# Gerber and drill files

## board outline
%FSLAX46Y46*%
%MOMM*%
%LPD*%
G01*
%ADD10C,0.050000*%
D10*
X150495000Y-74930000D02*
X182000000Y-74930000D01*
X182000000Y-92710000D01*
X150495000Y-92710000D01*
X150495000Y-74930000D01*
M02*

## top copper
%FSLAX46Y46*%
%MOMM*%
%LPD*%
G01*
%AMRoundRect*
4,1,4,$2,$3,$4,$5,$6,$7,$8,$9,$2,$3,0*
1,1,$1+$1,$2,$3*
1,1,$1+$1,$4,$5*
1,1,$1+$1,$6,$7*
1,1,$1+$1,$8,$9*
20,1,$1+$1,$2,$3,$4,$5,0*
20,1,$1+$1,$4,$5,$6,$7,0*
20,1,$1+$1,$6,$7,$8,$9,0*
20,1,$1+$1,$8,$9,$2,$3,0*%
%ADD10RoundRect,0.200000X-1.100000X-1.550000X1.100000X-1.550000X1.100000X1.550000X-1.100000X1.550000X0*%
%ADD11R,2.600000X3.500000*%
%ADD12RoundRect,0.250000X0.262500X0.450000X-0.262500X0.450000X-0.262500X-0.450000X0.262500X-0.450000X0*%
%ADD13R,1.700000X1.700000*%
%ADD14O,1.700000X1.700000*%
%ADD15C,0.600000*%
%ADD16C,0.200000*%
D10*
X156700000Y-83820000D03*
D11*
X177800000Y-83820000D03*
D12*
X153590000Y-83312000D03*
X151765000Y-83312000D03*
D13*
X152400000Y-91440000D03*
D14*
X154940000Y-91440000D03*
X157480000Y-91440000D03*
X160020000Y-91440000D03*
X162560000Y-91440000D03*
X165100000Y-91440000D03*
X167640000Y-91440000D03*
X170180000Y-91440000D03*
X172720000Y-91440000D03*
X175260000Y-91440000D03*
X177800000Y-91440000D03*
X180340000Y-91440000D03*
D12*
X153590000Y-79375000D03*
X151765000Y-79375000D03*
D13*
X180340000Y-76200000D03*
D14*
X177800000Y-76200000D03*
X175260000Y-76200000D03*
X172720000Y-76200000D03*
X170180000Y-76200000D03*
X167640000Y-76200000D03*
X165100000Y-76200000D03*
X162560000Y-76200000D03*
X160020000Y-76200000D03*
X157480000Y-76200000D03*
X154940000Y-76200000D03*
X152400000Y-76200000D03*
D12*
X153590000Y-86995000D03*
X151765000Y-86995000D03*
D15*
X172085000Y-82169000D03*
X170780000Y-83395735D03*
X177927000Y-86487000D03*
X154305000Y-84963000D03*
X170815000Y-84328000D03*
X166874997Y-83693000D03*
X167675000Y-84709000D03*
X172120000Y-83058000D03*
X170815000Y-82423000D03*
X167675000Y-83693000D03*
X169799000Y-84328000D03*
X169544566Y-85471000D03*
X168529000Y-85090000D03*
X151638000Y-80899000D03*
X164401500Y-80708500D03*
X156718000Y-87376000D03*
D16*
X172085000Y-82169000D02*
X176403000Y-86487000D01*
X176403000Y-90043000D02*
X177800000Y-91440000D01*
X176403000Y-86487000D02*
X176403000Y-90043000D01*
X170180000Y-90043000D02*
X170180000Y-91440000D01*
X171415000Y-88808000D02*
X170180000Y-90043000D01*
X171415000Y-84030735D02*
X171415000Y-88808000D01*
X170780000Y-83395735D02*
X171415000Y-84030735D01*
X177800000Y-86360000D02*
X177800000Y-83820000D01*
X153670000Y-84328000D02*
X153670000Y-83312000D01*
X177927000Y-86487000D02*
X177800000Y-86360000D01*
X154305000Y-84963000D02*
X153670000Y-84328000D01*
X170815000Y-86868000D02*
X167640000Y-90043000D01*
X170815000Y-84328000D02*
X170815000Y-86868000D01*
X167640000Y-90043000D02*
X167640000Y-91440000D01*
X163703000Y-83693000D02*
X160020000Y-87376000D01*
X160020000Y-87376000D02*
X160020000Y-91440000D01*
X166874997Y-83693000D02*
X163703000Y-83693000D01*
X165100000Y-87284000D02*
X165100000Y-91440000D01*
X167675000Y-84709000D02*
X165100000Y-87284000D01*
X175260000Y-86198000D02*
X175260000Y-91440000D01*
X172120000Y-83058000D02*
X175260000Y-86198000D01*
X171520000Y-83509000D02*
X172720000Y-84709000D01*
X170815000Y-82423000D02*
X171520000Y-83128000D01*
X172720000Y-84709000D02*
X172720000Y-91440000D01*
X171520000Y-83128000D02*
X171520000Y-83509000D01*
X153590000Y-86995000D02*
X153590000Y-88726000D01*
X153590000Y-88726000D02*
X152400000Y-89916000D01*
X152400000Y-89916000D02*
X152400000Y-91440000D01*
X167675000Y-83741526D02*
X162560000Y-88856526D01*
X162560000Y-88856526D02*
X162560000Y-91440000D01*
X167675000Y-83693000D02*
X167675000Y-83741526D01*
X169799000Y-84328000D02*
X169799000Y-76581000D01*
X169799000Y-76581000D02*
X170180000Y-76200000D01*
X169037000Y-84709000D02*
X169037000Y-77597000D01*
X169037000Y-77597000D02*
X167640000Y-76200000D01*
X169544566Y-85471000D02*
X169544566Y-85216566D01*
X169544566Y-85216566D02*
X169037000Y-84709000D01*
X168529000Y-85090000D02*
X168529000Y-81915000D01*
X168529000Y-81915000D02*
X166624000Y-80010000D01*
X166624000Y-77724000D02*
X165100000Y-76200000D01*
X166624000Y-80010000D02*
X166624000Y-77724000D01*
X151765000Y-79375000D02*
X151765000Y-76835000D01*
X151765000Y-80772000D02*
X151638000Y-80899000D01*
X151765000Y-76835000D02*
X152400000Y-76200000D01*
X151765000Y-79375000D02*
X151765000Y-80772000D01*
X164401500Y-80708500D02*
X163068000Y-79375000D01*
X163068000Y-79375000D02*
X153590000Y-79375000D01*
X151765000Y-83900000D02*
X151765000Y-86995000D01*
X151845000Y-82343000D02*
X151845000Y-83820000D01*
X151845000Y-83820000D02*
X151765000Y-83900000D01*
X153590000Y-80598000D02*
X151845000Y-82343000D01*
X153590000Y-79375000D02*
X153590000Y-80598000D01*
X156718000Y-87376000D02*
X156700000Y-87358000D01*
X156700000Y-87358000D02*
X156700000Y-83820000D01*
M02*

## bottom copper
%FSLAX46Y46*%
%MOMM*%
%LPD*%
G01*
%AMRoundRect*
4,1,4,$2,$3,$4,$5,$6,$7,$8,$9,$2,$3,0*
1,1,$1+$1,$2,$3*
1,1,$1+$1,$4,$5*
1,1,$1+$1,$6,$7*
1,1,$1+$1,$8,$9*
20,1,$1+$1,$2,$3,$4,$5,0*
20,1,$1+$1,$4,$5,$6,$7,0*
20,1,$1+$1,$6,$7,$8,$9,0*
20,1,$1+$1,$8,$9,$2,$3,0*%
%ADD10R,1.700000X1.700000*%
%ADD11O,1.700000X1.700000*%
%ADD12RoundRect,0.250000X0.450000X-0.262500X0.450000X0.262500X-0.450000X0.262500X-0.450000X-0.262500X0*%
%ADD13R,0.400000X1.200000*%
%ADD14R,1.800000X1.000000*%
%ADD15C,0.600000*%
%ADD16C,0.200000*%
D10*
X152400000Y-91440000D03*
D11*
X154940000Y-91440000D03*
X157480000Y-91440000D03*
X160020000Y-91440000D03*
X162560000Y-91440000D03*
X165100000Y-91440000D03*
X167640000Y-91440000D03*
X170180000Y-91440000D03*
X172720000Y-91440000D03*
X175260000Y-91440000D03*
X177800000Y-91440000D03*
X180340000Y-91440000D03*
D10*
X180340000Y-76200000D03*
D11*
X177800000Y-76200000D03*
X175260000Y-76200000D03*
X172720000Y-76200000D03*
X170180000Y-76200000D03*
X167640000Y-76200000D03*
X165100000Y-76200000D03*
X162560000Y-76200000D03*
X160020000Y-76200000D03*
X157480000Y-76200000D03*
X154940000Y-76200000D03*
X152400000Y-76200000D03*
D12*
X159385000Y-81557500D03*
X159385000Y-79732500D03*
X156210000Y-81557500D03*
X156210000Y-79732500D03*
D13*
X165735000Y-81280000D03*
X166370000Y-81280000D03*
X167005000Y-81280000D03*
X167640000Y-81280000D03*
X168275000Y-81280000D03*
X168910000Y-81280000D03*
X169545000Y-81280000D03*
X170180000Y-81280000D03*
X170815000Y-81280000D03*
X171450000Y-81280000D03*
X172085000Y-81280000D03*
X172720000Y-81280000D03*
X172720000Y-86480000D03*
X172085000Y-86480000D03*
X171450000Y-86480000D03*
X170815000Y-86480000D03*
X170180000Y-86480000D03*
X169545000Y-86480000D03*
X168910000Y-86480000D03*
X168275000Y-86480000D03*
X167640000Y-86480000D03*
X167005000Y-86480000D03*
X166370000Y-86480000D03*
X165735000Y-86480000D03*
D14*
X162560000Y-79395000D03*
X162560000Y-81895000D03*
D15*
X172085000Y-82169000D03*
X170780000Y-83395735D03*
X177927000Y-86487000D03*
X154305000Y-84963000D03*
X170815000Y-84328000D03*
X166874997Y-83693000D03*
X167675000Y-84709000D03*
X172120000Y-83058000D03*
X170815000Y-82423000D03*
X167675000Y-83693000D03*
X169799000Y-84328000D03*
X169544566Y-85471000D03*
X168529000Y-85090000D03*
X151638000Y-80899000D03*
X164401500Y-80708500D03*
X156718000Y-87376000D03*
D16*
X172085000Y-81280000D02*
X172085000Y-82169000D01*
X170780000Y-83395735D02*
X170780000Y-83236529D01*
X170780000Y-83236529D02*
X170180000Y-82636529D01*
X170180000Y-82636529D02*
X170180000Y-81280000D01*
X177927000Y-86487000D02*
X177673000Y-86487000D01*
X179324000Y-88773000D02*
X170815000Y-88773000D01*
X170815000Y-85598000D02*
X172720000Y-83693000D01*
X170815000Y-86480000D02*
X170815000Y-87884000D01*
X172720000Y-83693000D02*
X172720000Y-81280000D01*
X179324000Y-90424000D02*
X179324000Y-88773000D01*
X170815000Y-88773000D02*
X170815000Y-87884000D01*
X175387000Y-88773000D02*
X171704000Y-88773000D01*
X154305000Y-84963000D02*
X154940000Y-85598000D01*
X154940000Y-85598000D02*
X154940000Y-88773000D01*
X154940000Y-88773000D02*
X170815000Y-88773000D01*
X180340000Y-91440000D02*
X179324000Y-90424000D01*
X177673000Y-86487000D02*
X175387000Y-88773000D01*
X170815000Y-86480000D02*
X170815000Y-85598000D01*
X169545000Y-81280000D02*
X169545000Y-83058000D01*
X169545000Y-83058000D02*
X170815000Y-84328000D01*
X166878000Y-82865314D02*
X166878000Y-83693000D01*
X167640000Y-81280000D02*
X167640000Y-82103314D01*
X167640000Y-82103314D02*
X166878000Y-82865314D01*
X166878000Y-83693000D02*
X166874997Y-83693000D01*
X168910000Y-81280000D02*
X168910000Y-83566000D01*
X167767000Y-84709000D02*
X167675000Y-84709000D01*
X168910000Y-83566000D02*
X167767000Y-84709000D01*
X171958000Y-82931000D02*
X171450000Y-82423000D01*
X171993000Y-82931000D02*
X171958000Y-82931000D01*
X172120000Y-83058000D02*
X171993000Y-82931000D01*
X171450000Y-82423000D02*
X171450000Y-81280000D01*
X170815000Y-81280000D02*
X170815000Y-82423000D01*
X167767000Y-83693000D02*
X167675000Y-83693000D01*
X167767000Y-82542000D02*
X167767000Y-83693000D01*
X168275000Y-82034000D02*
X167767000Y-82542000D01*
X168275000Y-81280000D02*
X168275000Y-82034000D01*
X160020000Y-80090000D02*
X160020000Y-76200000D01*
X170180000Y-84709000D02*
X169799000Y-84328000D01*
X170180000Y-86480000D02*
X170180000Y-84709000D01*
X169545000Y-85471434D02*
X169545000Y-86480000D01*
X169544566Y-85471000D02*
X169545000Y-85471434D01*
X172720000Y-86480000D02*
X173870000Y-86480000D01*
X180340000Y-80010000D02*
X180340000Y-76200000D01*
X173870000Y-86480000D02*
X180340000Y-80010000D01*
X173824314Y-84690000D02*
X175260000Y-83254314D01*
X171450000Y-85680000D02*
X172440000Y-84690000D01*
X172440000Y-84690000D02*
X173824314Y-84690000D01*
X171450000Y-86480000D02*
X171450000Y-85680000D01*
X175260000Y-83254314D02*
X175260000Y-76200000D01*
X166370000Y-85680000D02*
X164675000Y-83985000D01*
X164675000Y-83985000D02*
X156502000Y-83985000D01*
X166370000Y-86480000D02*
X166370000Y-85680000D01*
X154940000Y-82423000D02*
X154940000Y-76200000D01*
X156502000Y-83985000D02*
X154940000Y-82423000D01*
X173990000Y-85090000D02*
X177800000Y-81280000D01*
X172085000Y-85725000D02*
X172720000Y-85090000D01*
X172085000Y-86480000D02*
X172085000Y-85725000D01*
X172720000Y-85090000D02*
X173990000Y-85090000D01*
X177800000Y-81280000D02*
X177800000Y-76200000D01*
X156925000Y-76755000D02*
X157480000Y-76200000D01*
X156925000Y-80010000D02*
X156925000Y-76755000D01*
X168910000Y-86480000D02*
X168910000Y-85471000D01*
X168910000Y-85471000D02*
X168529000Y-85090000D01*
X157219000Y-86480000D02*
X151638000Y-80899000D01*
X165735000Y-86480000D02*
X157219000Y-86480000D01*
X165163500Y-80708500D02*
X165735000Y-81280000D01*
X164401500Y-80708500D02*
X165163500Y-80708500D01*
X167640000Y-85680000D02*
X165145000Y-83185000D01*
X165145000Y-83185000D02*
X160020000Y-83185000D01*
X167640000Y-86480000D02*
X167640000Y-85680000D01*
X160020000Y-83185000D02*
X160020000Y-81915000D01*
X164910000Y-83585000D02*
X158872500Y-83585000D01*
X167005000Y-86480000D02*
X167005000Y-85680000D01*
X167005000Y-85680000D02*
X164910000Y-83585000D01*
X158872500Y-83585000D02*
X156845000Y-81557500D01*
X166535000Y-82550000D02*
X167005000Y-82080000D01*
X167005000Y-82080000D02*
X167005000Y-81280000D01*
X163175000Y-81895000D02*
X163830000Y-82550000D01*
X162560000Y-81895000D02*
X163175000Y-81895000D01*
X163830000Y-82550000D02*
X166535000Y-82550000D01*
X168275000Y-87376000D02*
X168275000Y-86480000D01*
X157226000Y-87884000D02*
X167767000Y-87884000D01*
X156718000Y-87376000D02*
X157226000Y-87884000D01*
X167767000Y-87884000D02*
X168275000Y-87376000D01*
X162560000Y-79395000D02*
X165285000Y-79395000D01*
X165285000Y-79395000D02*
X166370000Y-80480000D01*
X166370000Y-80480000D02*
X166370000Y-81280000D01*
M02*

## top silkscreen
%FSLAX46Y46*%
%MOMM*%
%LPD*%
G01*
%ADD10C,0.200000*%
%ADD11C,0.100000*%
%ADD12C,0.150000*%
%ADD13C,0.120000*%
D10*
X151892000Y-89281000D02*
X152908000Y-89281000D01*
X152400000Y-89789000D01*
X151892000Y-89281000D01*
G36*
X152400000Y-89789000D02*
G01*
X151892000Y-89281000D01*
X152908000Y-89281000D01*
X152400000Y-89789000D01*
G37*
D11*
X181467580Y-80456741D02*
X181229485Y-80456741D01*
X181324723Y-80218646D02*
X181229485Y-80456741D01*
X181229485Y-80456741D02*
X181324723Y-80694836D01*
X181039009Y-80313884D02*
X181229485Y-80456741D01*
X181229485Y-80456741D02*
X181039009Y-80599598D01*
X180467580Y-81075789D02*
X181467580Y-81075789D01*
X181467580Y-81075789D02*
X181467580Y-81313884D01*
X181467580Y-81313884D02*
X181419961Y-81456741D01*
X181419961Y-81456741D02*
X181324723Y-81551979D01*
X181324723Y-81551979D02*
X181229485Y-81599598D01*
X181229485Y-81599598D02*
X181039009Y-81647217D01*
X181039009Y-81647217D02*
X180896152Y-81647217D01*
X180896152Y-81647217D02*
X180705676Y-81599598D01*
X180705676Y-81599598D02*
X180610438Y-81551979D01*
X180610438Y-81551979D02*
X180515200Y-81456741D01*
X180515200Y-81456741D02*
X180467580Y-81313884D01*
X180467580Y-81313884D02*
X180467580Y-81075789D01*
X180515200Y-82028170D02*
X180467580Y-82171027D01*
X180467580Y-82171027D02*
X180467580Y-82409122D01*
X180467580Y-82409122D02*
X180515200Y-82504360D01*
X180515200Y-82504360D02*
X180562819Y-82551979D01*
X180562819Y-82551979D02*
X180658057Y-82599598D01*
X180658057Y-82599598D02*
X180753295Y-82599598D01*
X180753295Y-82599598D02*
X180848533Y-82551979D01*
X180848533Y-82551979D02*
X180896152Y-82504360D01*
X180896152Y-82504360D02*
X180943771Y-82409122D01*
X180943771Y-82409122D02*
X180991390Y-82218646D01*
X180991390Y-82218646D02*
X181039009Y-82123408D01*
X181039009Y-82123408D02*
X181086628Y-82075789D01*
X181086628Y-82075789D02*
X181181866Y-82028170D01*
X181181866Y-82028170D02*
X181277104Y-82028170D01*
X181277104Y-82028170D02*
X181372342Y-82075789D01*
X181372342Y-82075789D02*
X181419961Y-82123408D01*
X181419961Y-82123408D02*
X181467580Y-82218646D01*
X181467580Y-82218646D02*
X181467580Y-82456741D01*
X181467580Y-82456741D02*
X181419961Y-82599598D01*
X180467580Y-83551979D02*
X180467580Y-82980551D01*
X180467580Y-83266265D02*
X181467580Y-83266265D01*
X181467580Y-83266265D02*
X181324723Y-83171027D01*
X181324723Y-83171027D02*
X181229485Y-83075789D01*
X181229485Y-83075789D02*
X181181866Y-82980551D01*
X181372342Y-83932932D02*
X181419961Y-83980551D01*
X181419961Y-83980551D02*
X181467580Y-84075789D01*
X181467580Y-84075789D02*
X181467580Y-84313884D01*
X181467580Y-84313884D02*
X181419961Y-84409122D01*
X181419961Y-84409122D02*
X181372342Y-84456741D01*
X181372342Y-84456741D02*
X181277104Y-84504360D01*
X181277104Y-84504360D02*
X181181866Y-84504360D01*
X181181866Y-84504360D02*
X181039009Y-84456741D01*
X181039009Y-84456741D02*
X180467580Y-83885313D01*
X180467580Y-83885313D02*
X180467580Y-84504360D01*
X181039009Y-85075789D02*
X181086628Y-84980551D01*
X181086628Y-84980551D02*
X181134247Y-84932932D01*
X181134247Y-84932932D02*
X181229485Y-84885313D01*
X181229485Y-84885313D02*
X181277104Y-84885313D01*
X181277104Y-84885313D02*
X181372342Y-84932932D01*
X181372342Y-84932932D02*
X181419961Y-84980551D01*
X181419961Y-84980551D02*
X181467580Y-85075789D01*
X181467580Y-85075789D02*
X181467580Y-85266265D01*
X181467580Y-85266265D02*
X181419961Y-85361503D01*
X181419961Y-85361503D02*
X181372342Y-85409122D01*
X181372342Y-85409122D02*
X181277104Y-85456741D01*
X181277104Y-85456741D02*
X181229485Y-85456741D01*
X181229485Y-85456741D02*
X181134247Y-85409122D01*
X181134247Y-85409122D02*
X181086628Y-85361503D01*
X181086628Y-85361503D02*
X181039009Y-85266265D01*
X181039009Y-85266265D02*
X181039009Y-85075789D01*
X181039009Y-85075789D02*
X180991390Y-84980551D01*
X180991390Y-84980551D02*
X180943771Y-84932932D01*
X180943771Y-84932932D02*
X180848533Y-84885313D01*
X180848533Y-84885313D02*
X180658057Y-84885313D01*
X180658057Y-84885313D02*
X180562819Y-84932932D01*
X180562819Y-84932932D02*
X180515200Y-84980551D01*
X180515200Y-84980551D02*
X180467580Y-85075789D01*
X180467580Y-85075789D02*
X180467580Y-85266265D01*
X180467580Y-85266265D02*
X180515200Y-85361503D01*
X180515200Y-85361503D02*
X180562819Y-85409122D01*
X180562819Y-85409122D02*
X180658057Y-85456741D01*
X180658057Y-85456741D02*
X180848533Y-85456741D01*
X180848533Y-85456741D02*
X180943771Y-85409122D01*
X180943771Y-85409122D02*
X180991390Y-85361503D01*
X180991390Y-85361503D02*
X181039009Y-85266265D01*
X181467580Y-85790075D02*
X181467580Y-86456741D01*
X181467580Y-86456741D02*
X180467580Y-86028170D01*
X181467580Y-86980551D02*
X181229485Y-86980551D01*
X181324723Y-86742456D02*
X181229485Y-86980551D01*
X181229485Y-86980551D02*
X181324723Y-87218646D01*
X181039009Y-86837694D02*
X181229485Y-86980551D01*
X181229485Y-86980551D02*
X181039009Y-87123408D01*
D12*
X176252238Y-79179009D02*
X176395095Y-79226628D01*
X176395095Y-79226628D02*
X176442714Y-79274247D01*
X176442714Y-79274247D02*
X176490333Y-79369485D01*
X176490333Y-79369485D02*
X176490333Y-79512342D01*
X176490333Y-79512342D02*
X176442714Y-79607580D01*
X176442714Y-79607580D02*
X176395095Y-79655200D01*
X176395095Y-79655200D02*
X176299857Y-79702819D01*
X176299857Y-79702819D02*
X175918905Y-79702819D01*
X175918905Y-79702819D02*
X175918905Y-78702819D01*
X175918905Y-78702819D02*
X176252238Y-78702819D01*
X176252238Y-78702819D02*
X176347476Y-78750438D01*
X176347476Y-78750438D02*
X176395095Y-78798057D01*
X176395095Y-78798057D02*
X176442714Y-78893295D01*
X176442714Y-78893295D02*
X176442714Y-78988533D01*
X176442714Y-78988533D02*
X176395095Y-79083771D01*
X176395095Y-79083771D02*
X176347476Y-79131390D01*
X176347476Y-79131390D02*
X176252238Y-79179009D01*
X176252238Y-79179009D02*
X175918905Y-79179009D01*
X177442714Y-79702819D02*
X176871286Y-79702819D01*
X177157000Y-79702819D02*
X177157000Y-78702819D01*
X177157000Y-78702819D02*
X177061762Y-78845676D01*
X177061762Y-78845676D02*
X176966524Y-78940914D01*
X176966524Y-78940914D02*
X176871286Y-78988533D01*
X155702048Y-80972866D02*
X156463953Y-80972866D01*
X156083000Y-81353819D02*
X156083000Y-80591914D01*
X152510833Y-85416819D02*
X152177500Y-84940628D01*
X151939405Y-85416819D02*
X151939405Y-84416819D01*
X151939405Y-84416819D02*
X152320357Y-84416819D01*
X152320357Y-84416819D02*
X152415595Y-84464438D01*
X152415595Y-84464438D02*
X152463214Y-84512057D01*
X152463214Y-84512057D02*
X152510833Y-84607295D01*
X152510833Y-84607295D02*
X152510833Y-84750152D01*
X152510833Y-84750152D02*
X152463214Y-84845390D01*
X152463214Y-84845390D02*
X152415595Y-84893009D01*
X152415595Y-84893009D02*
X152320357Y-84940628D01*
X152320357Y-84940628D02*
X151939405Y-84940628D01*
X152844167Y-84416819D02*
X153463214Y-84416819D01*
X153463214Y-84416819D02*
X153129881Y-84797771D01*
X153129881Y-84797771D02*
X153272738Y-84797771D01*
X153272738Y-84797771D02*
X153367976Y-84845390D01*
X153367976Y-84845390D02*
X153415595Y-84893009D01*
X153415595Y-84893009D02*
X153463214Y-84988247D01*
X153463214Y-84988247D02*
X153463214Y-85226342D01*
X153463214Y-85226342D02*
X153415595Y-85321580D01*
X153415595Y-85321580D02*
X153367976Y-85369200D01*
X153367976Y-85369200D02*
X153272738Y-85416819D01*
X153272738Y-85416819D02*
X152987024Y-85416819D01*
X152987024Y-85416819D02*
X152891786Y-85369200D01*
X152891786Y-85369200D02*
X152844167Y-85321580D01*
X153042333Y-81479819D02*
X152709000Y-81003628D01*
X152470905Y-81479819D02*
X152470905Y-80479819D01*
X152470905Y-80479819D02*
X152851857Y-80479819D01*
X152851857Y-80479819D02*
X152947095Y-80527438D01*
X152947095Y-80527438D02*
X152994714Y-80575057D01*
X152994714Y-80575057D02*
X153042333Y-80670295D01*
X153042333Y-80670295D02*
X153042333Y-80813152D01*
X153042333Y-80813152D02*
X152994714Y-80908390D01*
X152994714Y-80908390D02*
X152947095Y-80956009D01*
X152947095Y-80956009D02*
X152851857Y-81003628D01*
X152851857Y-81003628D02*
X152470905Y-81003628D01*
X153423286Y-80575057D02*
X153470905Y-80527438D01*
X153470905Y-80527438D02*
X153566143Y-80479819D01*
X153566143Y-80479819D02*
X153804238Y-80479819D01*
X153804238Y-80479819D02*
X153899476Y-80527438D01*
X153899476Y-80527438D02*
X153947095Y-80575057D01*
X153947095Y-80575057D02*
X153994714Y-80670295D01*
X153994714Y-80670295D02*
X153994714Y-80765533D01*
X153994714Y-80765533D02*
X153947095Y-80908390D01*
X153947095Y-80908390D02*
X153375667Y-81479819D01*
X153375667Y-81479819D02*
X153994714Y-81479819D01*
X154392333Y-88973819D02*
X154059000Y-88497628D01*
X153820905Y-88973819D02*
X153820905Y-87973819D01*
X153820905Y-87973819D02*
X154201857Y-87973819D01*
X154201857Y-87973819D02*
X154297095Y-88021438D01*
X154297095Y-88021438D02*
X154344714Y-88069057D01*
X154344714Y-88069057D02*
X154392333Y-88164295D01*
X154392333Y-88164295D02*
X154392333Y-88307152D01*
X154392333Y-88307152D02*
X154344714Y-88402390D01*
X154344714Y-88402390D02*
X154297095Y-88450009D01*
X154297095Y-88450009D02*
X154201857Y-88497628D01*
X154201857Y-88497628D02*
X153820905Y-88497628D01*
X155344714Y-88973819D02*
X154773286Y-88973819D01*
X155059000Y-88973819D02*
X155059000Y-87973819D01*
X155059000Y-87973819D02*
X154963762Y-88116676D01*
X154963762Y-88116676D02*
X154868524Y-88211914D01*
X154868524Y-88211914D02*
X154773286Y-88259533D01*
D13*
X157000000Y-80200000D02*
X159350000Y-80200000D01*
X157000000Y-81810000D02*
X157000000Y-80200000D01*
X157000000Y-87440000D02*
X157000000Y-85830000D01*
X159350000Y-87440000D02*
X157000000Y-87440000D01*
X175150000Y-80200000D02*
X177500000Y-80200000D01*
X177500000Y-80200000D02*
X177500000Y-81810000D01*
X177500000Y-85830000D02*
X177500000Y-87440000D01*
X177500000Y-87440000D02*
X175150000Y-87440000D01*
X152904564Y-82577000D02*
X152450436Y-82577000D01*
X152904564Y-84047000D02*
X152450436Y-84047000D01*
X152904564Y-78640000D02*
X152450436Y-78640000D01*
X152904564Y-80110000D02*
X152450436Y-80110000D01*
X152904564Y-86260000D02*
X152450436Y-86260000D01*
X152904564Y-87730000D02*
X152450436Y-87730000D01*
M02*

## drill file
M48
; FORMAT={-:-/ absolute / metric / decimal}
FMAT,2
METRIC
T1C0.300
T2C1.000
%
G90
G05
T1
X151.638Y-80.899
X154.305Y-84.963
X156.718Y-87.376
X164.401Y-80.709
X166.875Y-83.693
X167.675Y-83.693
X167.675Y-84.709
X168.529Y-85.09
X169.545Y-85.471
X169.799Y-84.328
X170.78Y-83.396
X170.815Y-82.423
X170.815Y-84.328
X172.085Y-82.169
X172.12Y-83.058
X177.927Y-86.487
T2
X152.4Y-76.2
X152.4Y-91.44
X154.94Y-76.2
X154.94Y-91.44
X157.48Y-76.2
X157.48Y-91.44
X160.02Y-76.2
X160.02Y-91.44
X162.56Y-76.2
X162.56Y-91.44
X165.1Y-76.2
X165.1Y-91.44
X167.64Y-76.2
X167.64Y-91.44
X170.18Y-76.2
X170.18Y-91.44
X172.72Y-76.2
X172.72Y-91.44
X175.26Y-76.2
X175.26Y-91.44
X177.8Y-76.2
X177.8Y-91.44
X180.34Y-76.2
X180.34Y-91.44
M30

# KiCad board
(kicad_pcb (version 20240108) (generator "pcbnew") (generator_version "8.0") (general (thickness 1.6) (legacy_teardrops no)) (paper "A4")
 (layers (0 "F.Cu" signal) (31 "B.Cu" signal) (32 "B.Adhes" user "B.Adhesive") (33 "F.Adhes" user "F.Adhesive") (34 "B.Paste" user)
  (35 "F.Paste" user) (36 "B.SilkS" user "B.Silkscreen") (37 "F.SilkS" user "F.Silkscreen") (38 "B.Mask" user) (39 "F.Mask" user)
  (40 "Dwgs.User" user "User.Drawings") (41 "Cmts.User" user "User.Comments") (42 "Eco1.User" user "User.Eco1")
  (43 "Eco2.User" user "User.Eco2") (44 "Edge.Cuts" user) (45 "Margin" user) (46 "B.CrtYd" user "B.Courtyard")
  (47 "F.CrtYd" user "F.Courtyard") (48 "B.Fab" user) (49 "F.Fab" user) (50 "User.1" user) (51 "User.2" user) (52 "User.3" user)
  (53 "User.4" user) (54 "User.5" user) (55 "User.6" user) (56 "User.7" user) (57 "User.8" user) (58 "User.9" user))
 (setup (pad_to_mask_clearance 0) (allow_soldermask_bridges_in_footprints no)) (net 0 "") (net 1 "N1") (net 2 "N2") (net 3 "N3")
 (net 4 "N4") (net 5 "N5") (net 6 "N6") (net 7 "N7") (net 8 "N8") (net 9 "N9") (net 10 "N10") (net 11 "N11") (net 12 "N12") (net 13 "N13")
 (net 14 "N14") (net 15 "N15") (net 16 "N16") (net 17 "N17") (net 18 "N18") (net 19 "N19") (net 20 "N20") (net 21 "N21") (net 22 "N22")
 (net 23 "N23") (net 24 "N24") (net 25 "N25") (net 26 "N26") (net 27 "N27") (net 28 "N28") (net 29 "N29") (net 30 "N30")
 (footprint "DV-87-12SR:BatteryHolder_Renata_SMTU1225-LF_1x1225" (layer "F.Cu") (at 167.25 83.82)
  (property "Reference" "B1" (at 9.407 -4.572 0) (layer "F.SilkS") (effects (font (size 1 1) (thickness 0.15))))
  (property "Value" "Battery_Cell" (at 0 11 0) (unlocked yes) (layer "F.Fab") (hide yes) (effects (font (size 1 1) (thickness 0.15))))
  (fp_line (start -10.25 -3.62) (end -7.9 -3.62) (stroke (width 0.12) (type solid)) (layer "F.SilkS"))
  (fp_line (start -10.25 -2.01) (end -10.25 -3.62) (stroke (width 0.12) (type solid)) (layer "F.SilkS"))
  (fp_line (start -10.25 3.62) (end -10.25 2.01) (stroke (width 0.12) (type solid)) (layer "F.SilkS"))
  (fp_line (start -7.9 3.62) (end -10.25 3.62) (stroke (width 0.12) (type solid)) (layer "F.SilkS"))
  (fp_line (start 7.9 -3.62) (end 10.25 -3.62) (stroke (width 0.12) (type solid)) (layer "F.SilkS"))
  (fp_line (start 10.25 -3.62) (end 10.25 -2.01) (stroke (width 0.12) (type solid)) (layer "F.SilkS"))
  (fp_line (start 10.25 2.01) (end 10.25 3.62) (stroke (width 0.12) (type solid)) (layer "F.SilkS"))
  (fp_line (start 10.25 3.62) (end 7.9 3.62) (stroke (width 0.12) (type solid)) (layer "F.SilkS"))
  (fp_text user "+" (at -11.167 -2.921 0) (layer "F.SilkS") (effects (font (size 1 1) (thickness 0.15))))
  (pad "1" smd roundrect (at -10.55 0) (size 2.6 3.5) (layers "F.Cu" "F.Paste" "F.Mask") (roundrect_rratio 0.07692307692) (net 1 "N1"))
  (pad "2" smd rect (at 10.55 0) (size 2.6 3.5) (layers "F.Cu" "F.Paste" "F.Mask") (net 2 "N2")))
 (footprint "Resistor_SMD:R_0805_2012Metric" (layer "F.Cu") (at 152.6775 83.312 180)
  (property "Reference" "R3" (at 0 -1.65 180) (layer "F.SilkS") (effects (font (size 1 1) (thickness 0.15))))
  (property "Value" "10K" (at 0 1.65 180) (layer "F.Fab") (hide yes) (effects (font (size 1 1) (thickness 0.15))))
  (fp_line (start -0.227064 0.735) (end 0.227064 0.735) (stroke (width 0.12) (type solid)) (layer "F.SilkS"))
  (fp_line (start -0.227064 -0.735) (end 0.227064 -0.735) (stroke (width 0.12) (type solid)) (layer "F.SilkS"))
  (pad "1" smd roundrect (at -0.9125 0 180) (size 1.025 1.4) (layers "F.Cu" "F.Paste" "F.Mask") (roundrect_rratio 0.243902) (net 2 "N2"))
  (pad "2" smd roundrect (at 0.9125 0 180) (size 1.025 1.4) (layers "F.Cu" "F.Paste" "F.Mask") (roundrect_rratio 0.243902) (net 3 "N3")))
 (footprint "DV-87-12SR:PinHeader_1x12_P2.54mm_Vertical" (layer "F.Cu") (at 152.4 91.44 90)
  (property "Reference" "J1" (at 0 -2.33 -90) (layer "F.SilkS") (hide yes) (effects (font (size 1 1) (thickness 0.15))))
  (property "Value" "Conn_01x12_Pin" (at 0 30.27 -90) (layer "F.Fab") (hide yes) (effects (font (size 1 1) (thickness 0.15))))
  (pad "1" thru_hole rect (at 0 0 90) (size 1.7 1.7) (drill 1) (layers "*.Cu" "*.Mask") (remove_unused_layers no) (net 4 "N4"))
  (pad "2" thru_hole oval (at 0 2.54 90) (size 1.7 1.7) (drill 1) (layers "*.Cu" "*.Mask") (remove_unused_layers no) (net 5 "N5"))
  (pad "3" thru_hole oval (at 0 5.08 90) (size 1.7 1.7) (drill 1) (layers "*.Cu" "*.Mask") (remove_unused_layers no) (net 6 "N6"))
  (pad "4" thru_hole oval (at 0 7.62 90) (size 1.7 1.7) (drill 1) (layers "*.Cu" "*.Mask") (remove_unused_layers no) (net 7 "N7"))
  (pad "5" thru_hole oval (at 0 10.16 90) (size 1.7 1.7) (drill 1) (layers "*.Cu" "*.Mask") (remove_unused_layers no) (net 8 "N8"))
  (pad "6" thru_hole oval (at 0 12.7 90) (size 1.7 1.7) (drill 1) (layers "*.Cu" "*.Mask") (remove_unused_layers no) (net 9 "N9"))
  (pad "7" thru_hole oval (at 0 15.24 90) (size 1.7 1.7) (drill 1) (layers "*.Cu" "*.Mask") (remove_unused_layers no) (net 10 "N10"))
  (pad "8" thru_hole oval (at 0 17.78 90) (size 1.7 1.7) (drill 1) (layers "*.Cu" "*.Mask") (remove_unused_layers no) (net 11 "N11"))
  (pad "9" thru_hole oval (at 0 20.32 90) (size 1.7 1.7) (drill 1) (layers "*.Cu" "*.Mask") (remove_unused_layers no) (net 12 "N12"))
  (pad "10" thru_hole oval (at 0 22.86 90) (size 1.7 1.7) (drill 1) (layers "*.Cu" "*.Mask") (remove_unused_layers no) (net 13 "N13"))
  (pad "11" thru_hole oval (at 0 25.4 90) (size 1.7 1.7) (drill 1) (layers "*.Cu" "*.Mask") (remove_unused_layers no) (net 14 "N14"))
  (pad "12" thru_hole oval (at 0 27.94 90) (size 1.7 1.7) (drill 1) (layers "*.Cu" "*.Mask") (remove_unused_layers no) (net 2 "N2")))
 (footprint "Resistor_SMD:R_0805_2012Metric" (layer "F.Cu") (at 152.6775 79.375 180)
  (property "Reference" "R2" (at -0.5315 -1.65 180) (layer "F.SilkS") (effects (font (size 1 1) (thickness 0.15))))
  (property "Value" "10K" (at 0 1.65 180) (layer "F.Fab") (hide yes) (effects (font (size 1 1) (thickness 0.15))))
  (fp_line (start -0.227064 0.735) (end 0.227064 0.735) (stroke (width 0.12) (type solid)) (layer "F.SilkS"))
  (fp_line (start -0.227064 -0.735) (end 0.227064 -0.735) (stroke (width 0.12) (type solid)) (layer "F.SilkS"))
  (pad "1" smd roundrect (at -0.9125 0 180) (size 1.025 1.4) (layers "F.Cu" "F.Paste" "F.Mask") (roundrect_rratio 0.243902) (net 3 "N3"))
  (pad "2" smd roundrect (at 0.9125 0 180) (size 1.025 1.4) (layers "F.Cu" "F.Paste" "F.Mask") (roundrect_rratio 0.243902) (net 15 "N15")))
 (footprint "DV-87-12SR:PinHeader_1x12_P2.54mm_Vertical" (layer "F.Cu") (at 180.34 76.2 -90)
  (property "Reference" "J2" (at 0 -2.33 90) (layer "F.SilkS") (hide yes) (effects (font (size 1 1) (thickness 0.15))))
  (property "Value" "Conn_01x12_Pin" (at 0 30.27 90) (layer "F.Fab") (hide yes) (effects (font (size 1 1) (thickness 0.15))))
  (pad "1" thru_hole rect (at 0 0 270) (size 1.7 1.7) (drill 1) (layers "*.Cu" "*.Mask") (remove_unused_layers no) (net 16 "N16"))
  (pad "2" thru_hole oval (at 0 2.54 270) (size 1.7 1.7) (drill 1) (layers "*.Cu" "*.Mask") (remove_unused_layers no) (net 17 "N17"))
  (pad "3" thru_hole oval (at 0 5.08 270) (size 1.7 1.7) (drill 1) (layers "*.Cu" "*.Mask") (remove_unused_layers no) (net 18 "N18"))
  (pad "4" thru_hole oval (at 0 7.62 270) (size 1.7 1.7) (drill 1) (layers "*.Cu" "*.Mask") (remove_unused_layers no) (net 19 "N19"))
  (pad "5" thru_hole oval (at 0 10.16 270) (size 1.7 1.7) (drill 1) (layers "*.Cu" "*.Mask") (remove_unused_layers no) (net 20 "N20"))
  (pad "6" thru_hole oval (at 0 12.7 270) (size 1.7 1.7) (drill 1) (layers "*.Cu" "*.Mask") (remove_unused_layers no) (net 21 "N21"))
  (pad "7" thru_hole oval (at 0 15.24 270) (size 1.7 1.7) (drill 1) (layers "*.Cu" "*.Mask") (remove_unused_layers no) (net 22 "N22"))
  (pad "8" thru_hole oval (at 0 17.78 270) (size 1.7 1.7) (drill 1) (layers "*.Cu" "*.Mask") (remove_unused_layers no) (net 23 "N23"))
  (pad "9" thru_hole oval (at 0 20.32 270) (size 1.7 1.7) (drill 1) (layers "*.Cu" "*.Mask") (remove_unused_layers no) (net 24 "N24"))
  (pad "10" thru_hole oval (at 0 22.86 270) (size 1.7 1.7) (drill 1) (layers "*.Cu" "*.Mask") (remove_unused_layers no) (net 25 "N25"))
  (pad "11" thru_hole oval (at 0 25.4 270) (size 1.7 1.7) (drill 1) (layers "*.Cu" "*.Mask") (remove_unused_layers no) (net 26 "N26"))
  (pad "12" thru_hole oval (at 0 27.94 270) (size 1.7 1.7) (drill 1) (layers "*.Cu" "*.Mask") (remove_unused_layers no) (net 15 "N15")))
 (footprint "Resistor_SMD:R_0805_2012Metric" (layer "F.Cu") (at 152.6775 86.995 180)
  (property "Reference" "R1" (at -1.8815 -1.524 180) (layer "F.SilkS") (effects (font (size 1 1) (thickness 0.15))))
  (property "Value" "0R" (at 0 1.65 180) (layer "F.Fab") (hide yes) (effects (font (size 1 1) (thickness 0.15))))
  (fp_line (start -0.227064 0.735) (end 0.227064 0.735) (stroke (width 0.12) (type solid)) (layer "F.SilkS"))
  (fp_line (start -0.227064 -0.735) (end 0.227064 -0.735) (stroke (width 0.12) (type solid)) (layer "F.SilkS"))
  (pad "1" smd roundrect (at -0.9125 0 180) (size 1.025 1.4) (layers "F.Cu" "F.Paste" "F.Mask") (roundrect_rratio 0.243902) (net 4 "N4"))
  (pad "2" smd roundrect (at 0.9125 0 180) (size 1.025 1.4) (layers "F.Cu" "F.Paste" "F.Mask") (roundrect_rratio 0.243902) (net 3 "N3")))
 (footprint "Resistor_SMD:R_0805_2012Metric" (layer "B.Cu") (at 159.385 80.645 90)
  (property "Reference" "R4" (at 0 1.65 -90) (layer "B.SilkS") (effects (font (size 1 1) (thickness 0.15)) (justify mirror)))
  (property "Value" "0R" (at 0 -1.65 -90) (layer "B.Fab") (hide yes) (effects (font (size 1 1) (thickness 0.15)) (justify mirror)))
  (pad "1" smd roundrect (at -0.9125 0 90) (size 1.025 1.4) (layers "B.Cu" "B.Paste" "B.Mask") (roundrect_rratio 0.243902) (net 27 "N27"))
  (pad "2" smd roundrect (at 0.9125 0 90) (size 1.025 1.4) (layers "B.Cu" "B.Paste" "B.Mask") (roundrect_rratio 0.243902) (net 24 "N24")))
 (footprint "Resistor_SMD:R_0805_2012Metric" (layer "B.Cu") (at 156.21 80.645 90)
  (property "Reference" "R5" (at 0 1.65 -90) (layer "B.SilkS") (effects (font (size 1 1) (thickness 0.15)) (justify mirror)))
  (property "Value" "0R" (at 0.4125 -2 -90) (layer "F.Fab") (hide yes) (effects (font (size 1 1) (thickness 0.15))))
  (pad "1" smd roundrect (at -0.9125 0 90) (size 1.025 1.4) (layers "B.Cu" "B.Paste" "B.Mask") (roundrect_rratio 0.243902) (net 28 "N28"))
  (pad "2" smd roundrect (at 0.9125 0 90) (size 1.025 1.4) (layers "B.Cu" "B.Paste" "B.Mask") (roundrect_rratio 0.243902) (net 25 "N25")))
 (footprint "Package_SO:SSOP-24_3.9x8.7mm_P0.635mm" (layer "B.Cu") (at 169.2275 83.88 -90)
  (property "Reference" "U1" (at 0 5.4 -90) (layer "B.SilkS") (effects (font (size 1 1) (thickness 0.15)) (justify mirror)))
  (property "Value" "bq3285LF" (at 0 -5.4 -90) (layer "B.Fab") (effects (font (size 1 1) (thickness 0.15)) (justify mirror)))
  (pad "1" smd rect (at -2.6 3.4925 270) (size 1.2 0.4) (layers "B.Cu" "B.Paste" "B.Mask") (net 3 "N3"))
  (pad "2" smd rect (at -2.6 2.8575 270) (size 1.2 0.4) (layers "B.Cu" "B.Paste" "B.Mask") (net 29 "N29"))
  (pad "3" smd rect (at -2.6 2.2225 270) (size 1.2 0.4) (layers "B.Cu" "B.Paste" "B.Mask") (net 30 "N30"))
  (pad "4" smd rect (at -2.6 1.5875 270) (size 1.2 0.4) (layers "B.Cu" "B.Paste" "B.Mask") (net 7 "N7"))
  (pad "5" smd rect (at -2.6 0.9525 270) (size 1.2 0.4) (layers "B.Cu" "B.Paste" "B.Mask") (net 8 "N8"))
  (pad "6" smd rect (at -2.6 0.3175 270) (size 1.2 0.4) (layers "B.Cu" "B.Paste" "B.Mask") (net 9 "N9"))
  (pad "7" smd rect (at -2.6 -0.3175 270) (size 1.2 0.4) (layers "B.Cu" "B.Paste" "B.Mask") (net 10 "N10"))
  (pad "8" smd rect (at -2.6 -0.9525 270) (size 1.2 0.4) (layers "B.Cu" "B.Paste" "B.Mask") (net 11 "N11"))
  (pad "9" smd rect (at -2.6 -1.5875 270) (size 1.2 0.4) (layers "B.Cu" "B.Paste" "B.Mask") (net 12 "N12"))
  (pad "10" smd rect (at -2.6 -2.2225 270) (size 1.2 0.4) (layers "B.Cu" "B.Paste" "B.Mask") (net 13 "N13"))
  (pad "11" smd rect (at -2.6 -2.8575 270) (size 1.2 0.4) (layers "B.Cu" "B.Paste" "B.Mask") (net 14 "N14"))
  (pad "12" smd rect (at -2.6 -3.4925 270) (size 1.2 0.4) (layers "B.Cu" "B.Paste" "B.Mask") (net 2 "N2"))
  (pad "13" smd rect (at 2.6 -3.4925 270) (size 1.2 0.4) (layers "B.Cu" "B.Paste" "B.Mask") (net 16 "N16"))
  (pad "14" smd rect (at 2.6 -2.8575 270) (size 1.2 0.4) (layers "B.Cu" "B.Paste" "B.Mask") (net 17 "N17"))
  (pad "15" smd rect (at 2.6 -2.2225 270) (size 1.2 0.4) (layers "B.Cu" "B.Paste" "B.Mask") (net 18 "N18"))
  (pad "16" smd rect (at 2.6 -1.5875 270) (size 1.2 0.4) (layers "B.Cu" "B.Paste" "B.Mask") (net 2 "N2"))
  (pad "17" smd rect (at 2.6 -0.9525 270) (size 1.2 0.4) (layers "B.Cu" "B.Paste" "B.Mask") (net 20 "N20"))
  (pad "18" smd rect (at 2.6 -0.3175 270) (size 1.2 0.4) (layers "B.Cu" "B.Paste" "B.Mask") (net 21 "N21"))
  (pad "19" smd rect (at 2.6 0.3175 270) (size 1.2 0.4) (layers "B.Cu" "B.Paste" "B.Mask") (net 22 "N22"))
  (pad "20" smd rect (at 2.6 0.9525 270) (size 1.2 0.4) (layers "B.Cu" "B.Paste" "B.Mask") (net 1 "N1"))
  (pad "21" smd rect (at 2.6 1.5875 270) (size 1.2 0.4) (layers "B.Cu" "B.Paste" "B.Mask") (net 27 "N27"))
  (pad "22" smd rect (at 2.6 2.2225 270) (size 1.2 0.4) (layers "B.Cu" "B.Paste" "B.Mask") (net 28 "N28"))
  (pad "23" smd rect (at 2.6 2.8575 270) (size 1.2 0.4) (layers "B.Cu" "B.Paste" "B.Mask") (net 26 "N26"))
  (pad "24" smd rect (at 2.6 3.4925 270) (size 1.2 0.4) (layers "B.Cu" "B.Paste" "B.Mask") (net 15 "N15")))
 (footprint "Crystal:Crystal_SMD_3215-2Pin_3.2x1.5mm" (layer "B.Cu") (at 162.56 80.645 90)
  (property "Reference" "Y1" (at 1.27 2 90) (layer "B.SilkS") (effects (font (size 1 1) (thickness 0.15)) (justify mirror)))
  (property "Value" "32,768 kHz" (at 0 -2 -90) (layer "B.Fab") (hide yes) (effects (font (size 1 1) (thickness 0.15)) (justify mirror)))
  (pad "1" smd rect (at 1.25 0 90) (size 1 1.8) (layers "B.Cu" "B.Paste" "B.Mask") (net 29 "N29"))
  (pad "2" smd rect (at -1.25 0 90) (size 1 1.8) (layers "B.Cu" "B.Paste" "B.Mask") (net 30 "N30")))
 (gr_poly (pts (xy 151.892 89.281) (xy 152.908 89.281) (xy 152.4 89.789)) (stroke (width 0.2) (type solid)) (fill solid) (layer "F.SilkS"))
 (gr_rect (start 150.495 74.93) (end 182 92.71) (stroke (width 0.05) (type default)) (fill none) (layer "Edge.Cuts"))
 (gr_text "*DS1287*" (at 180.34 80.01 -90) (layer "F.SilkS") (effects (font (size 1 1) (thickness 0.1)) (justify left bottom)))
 (segment (start 172.085 82.169) (end 176.403 86.487) (width 0.2) (layer "F.Cu") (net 14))
 (segment (start 176.403 90.043) (end 177.8 91.44) (width 0.2) (layer "F.Cu") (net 14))
 (segment (start 176.403 86.487) (end 176.403 90.043) (width 0.2) (layer "F.Cu") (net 14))
 (via (at 172.085 82.169) (size 0.6) (drill 0.3) (layers "F.Cu" "B.Cu") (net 14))
 (segment (start 172.085 81.28) (end 172.085 82.169) (width 0.2) (layer "B.Cu") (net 14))
 (segment (start 170.18 90.043) (end 170.18 91.44) (width 0.2) (layer "F.Cu") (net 11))
 (segment (start 171.415 88.808) (end 170.18 90.043) (width 0.2) (layer "F.Cu") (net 11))
 (segment (start 171.415 84.030735) (end 171.415 88.808) (width 0.2) (layer "F.Cu") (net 11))
 (segment (start 170.78 83.395735) (end 171.415 84.030735) (width 0.2) (layer "F.Cu") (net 11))
 (via (at 170.78 83.395735) (size 0.6) (drill 0.3) (layers "F.Cu" "B.Cu") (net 11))
 (segment (start 170.78 83.395735) (end 170.78 83.236529) (width 0.2) (layer "B.Cu") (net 11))
 (segment (start 170.78 83.236529) (end 170.18 82.636529) (width 0.2) (layer "B.Cu") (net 11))
 (segment (start 170.18 82.636529) (end 170.18 81.28) (width 0.2) (layer "B.Cu") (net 11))
 (segment (start 177.8 86.36) (end 177.8 83.82) (width 0.2) (layer "F.Cu") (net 2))
 (segment (start 153.67 84.328) (end 153.67 83.312) (width 0.2) (layer "F.Cu") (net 2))
 (segment (start 177.927 86.487) (end 177.8 86.36) (width 0.2) (layer "F.Cu") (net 2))
 (segment (start 154.305 84.963) (end 153.67 84.328) (width 0.2) (layer "F.Cu") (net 2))
 (via (at 177.927 86.487) (size 0.6) (drill 0.3) (layers "F.Cu" "B.Cu") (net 2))
 (via (at 154.305 84.963) (size 0.6) (drill 0.3) (layers "F.Cu" "B.Cu") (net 2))
 (segment (start 177.927 86.487) (end 177.673 86.487) (width 0.2) (layer "B.Cu") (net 2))
 (segment (start 179.324 88.773) (end 170.815 88.773) (width 0.2) (layer "B.Cu") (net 2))
 (segment (start 170.815 85.598) (end 172.72 83.693) (width 0.2) (layer "B.Cu") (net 2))
 (segment (start 170.815 86.48) (end 170.815 87.884) (width 0.2) (layer "B.Cu") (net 2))
 (segment (start 172.72 83.693) (end 172.72 81.28) (width 0.2) (layer "B.Cu") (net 2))
 (segment (start 179.324 90.424) (end 179.324 88.773) (width 0.2) (layer "B.Cu") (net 2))
 (segment (start 170.815 88.773) (end 170.815 87.884) (width 0.2) (layer "B.Cu") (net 2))
 (segment (start 175.387 88.773) (end 171.704 88.773) (width 0.2) (layer "B.Cu") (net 2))
 (segment (start 154.305 84.963) (end 154.94 85.598) (width 0.2) (layer "B.Cu") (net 2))
 (segment (start 154.94 85.598) (end 154.94 88.773) (width 0.2) (layer "B.Cu") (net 2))
 (segment (start 154.94 88.773) (end 170.815 88.773) (width 0.2) (layer "B.Cu") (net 2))
 (segment (start 180.34 91.44) (end 179.324 90.424) (width 0.2) (layer "B.Cu") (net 2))
 (segment (start 177.673 86.487) (end 175.387 88.773) (width 0.2) (layer "B.Cu") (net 2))
 (segment (start 170.815 86.48) (end 170.815 85.598) (width 0.2) (layer "B.Cu") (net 2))
 (segment (start 170.815 86.868) (end 167.64 90.043) (width 0.2) (layer "F.Cu") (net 10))
 (segment (start 170.815 84.328) (end 170.815 86.868) (width 0.2) (layer "F.Cu") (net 10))
 (segment (start 167.64 90.043) (end 167.64 91.44) (width 0.2) (layer "F.Cu") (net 10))
 (via (at 170.815 84.328) (size 0.6) (drill 0.3) (layers "F.Cu" "B.Cu") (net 10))
 (segment (start 169.545 81.28) (end 169.545 83.058) (width 0.2) (layer "B.Cu") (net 10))
 (segment (start 169.545 83.058) (end 170.815 84.328) (width 0.2) (layer "B.Cu") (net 10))
 (segment (start 163.703 83.693) (end 160.02 87.376) (width 0.2) (layer "F.Cu") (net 7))
 (segment (start 160.02 87.376) (end 160.02 91.44) (width 0.2) (layer "F.Cu") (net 7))
 (segment (start 166.874997 83.693) (end 163.703 83.693) (width 0.2) (layer "F.Cu") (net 7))
 (via (at 166.874997 83.693) (size 0.6) (drill 0.3) (layers "F.Cu" "B.Cu") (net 7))
 (segment (start 166.878 82.865314) (end 166.878 83.693) (width 0.2) (layer "B.Cu") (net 7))
 (segment (start 167.64 81.28) (end 167.64 82.103314) (width 0.2) (layer "B.Cu") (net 7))
 (segment (start 167.64 82.103314) (end 166.878 82.865314) (width 0.2) (layer "B.Cu") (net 7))
 (segment (start 166.878 83.693) (end 166.874997 83.693) (width 0.2) (layer "B.Cu") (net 7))
 (segment (start 165.1 87.284) (end 165.1 91.44) (width 0.2) (layer "F.Cu") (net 9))
 (segment (start 167.675 84.709) (end 165.1 87.284) (width 0.2) (layer "F.Cu") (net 9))
 (via (at 167.675 84.709) (size 0.6) (drill 0.3) (layers "F.Cu" "B.Cu") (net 9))
 (segment (start 168.91 81.28) (end 168.91 83.566) (width 0.2) (layer "B.Cu") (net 9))
 (segment (start 167.767 84.709) (end 167.675 84.709) (width 0.2) (layer "B.Cu") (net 9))
 (segment (start 168.91 83.566) (end 167.767 84.709) (width 0.2) (layer "B.Cu") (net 9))
 (segment (start 175.26 86.198) (end 175.26 91.44) (width 0.2) (layer "F.Cu") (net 13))
 (segment (start 172.12 83.058) (end 175.26 86.198) (width 0.2) (layer "F.Cu") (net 13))
 (via (at 172.12 83.058) (size 0.6) (drill 0.3) (layers "F.Cu" "B.Cu") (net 13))
 (segment (start 171.958 82.931) (end 171.45 82.423) (width 0.2) (layer "B.Cu") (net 13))
 (segment (start 171.993 82.931) (end 171.958 82.931) (width 0.2) (layer "B.Cu") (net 13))
 (segment (start 172.12 83.058) (end 171.993 82.931) (width 0.2) (layer "B.Cu") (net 13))
 (segment (start 171.45 82.423) (end 171.45 81.28) (width 0.2) (layer "B.Cu") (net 13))
 (segment (start 171.52 83.509) (end 172.72 84.709) (width 0.2) (layer "F.Cu") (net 12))
 (segment (start 170.815 82.423) (end 171.52 83.128) (width 0.2) (layer "F.Cu") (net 12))
 (segment (start 172.72 84.709) (end 172.72 91.44) (width 0.2) (layer "F.Cu") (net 12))
 (segment (start 171.52 83.128) (end 171.52 83.509) (width 0.2) (layer "F.Cu") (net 12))
 (via (at 170.815 82.423) (size 0.6) (drill 0.3) (layers "F.Cu" "B.Cu") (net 12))
 (segment (start 170.815 81.28) (end 170.815 82.423) (width 0.2) (layer "B.Cu") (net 12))
 (segment (start 153.59 86.995) (end 153.59 88.726) (width 0.2) (layer "F.Cu") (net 4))
 (segment (start 153.59 88.726) (end 152.4 89.916) (width 0.2) (layer "F.Cu") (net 4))
 (segment (start 152.4 89.916) (end 152.4 91.44) (width 0.2) (layer "F.Cu") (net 4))
 (segment (start 167.675 83.741526) (end 162.56 88.856526) (width 0.2) (layer "F.Cu") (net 8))
 (segment (start 162.56 88.856526) (end 162.56 91.44) (width 0.2) (layer "F.Cu") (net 8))
 (segment (start 167.675 83.693) (end 167.675 83.741526) (width 0.2) (layer "F.Cu") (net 8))
 (via (at 167.675 83.693) (size 0.6) (drill 0.3) (layers "F.Cu" "B.Cu") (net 8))
 (segment (start 167.767 83.693) (end 167.675 83.693) (width 0.2) (layer "B.Cu") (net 8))
 (segment (start 167.767 82.542) (end 167.767 83.693) (width 0.2) (layer "B.Cu") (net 8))
 (segment (start 168.275 82.034) (end 167.767 82.542) (width 0.2) (layer "B.Cu") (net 8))
 (segment (start 168.275 81.28) (end 168.275 82.034) (width 0.2) (layer "B.Cu") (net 8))
 (segment (start 160.02 80.09) (end 160.02 76.2) (width 0.2) (layer "B.Cu") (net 24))
 (segment (start 169.799 84.328) (end 169.799 76.581) (width 0.2) (layer "F.Cu") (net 20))
 (segment (start 169.799 76.581) (end 170.18 76.2) (width 0.2) (layer "F.Cu") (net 20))
 (via (at 169.799 84.328) (size 0.6) (drill 0.3) (layers "F.Cu" "B.Cu") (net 20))
 (segment (start 170.18 84.709) (end 169.799 84.328) (width 0.2) (layer "B.Cu") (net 20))
 (segment (start 170.18 86.48) (end 170.18 84.709) (width 0.2) (layer "B.Cu") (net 20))
 (segment (start 169.037 84.709) (end 169.037 77.597) (width 0.2) (layer "F.Cu") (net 21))
 (segment (start 169.037 77.597) (end 167.64 76.2) (width 0.2) (layer "F.Cu") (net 21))
 (segment (start 169.544566 85.471) (end 169.544566 85.216566) (width 0.2) (layer "F.Cu") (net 21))
 (segment (start 169.544566 85.216566) (end 169.037 84.709) (width 0.2) (layer "F.Cu") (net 21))
 (via (at 169.544566 85.471) (size 0.6) (drill 0.3) (layers "F.Cu" "B.Cu") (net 21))
 (segment (start 169.545 85.471434) (end 169.545 86.48) (width 0.2) (layer "B.Cu") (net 21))
 (segment (start 169.544566 85.471) (end 169.545 85.471434) (width 0.2) (layer "B.Cu") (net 21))
 (segment (start 172.72 86.48) (end 173.87 86.48) (width 0.2) (layer "B.Cu") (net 16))
 (segment (start 180.34 80.01) (end 180.34 76.2) (width 0.2) (layer "B.Cu") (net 16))
 (segment (start 173.87 86.48) (end 180.34 80.01) (width 0.2) (layer "B.Cu") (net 16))
 (segment (start 173.824314 84.69) (end 175.26 83.254314) (width 0.2) (layer "B.Cu") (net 18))
 (segment (start 171.45 85.68) (end 172.44 84.69) (width 0.2) (layer "B.Cu") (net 18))
 (segment (start 172.44 84.69) (end 173.824314 84.69) (width 0.2) (layer "B.Cu") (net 18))
 (segment (start 171.45 86.48) (end 171.45 85.68) (width 0.2) (layer "B.Cu") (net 18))
 (segment (start 175.26 83.254314) (end 175.26 76.2) (width 0.2) (layer "B.Cu") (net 18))
 (segment (start 166.37 85.68) (end 164.675 83.985) (width 0.2) (layer "B.Cu") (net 26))
 (segment (start 164.675 83.985) (end 156.502 83.985) (width 0.2) (layer "B.Cu") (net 26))
 (segment (start 166.37 86.48) (end 166.37 85.68) (width 0.2) (layer "B.Cu") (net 26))
 (segment (start 154.94 82.423) (end 154.94 76.2) (width 0.2) (layer "B.Cu") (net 26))
 (segment (start 156.502 83.985) (end 154.94 82.423) (width 0.2) (layer "B.Cu") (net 26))
 (segment (start 173.99 85.09) (end 177.8 81.28) (width 0.2) (layer "B.Cu") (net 17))
 (segment (start 172.085 85.725) (end 172.72 85.09) (width 0.2) (layer "B.Cu") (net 17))
 (segment (start 172.085 86.48) (end 172.085 85.725) (width 0.2) (layer "B.Cu") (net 17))
 (segment (start 172.72 85.09) (end 173.99 85.09) (width 0.2) (layer "B.Cu") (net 17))
 (segment (start 177.8 81.28) (end 177.8 76.2) (width 0.2) (layer "B.Cu") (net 17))
 (segment (start 156.925 76.755) (end 157.48 76.2) (width 0.2) (layer "B.Cu") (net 25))
 (segment (start 156.925 80.01) (end 156.925 76.755) (width 0.2) (layer "B.Cu") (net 25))
 (segment (start 168.529 85.09) (end 168.529 81.915) (width 0.2) (layer "F.Cu") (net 22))
 (segment (start 168.529 81.915) (end 166.624 80.01) (width 0.2) (layer "F.Cu") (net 22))
 (segment (start 166.624 77.724) (end 165.1 76.2) (width 0.2) (layer "F.Cu") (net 22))
 (segment (start 166.624 80.01) (end 166.624 77.724) (width 0.2) (layer "F.Cu") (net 22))
 (via (at 168.529 85.09) (size 0.6) (drill 0.3) (layers "F.Cu" "B.Cu") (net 22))
 (segment (start 168.91 86.48) (end 168.91 85.471) (width 0.2) (layer "B.Cu") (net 22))
 (segment (start 168.91 85.471) (end 168.529 85.09) (width 0.2) (layer "B.Cu") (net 22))
 (segment (start 151.765 79.375) (end 151.765 76.835) (width 0.2) (layer "F.Cu") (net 15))
 (segment (start 151.765 80.772) (end 151.638 80.899) (width 0.2) (layer "F.Cu") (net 15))
 (segment (start 151.765 76.835) (end 152.4 76.2) (width 0.2) (layer "F.Cu") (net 15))
 (segment (start 151.765 79.375) (end 151.765 80.772) (width 0.2) (layer "F.Cu") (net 15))
 (via (at 151.638 80.899) (size 0.6) (drill 0.3) (layers "F.Cu" "B.Cu") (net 15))
 (segment (start 157.219 86.48) (end 151.638 80.899) (width 0.2) (layer "B.Cu") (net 15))
 (segment (start 165.735 86.48) (end 157.219 86.48) (width 0.2) (layer "B.Cu") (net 15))
 (segment (start 164.4015 80.7085) (end 163.068 79.375) (width 0.2) (layer "F.Cu") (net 3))
 (segment (start 163.068 79.375) (end 153.59 79.375) (width 0.2) (layer "F.Cu") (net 3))
 (segment (start 151.765 83.9) (end 151.765 86.995) (width 0.2) (layer "F.Cu") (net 3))
 (segment (start 151.845 82.343) (end 151.845 83.82) (width 0.2) (layer "F.Cu") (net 3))
 (segment (start 151.845 83.82) (end 151.765 83.9) (width 0.2) (layer "F.Cu") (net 3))
 (segment (start 153.59 80.598) (end 151.845 82.343) (width 0.2) (layer "F.Cu") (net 3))
 (segment (start 153.59 79.375) (end 153.59 80.598) (width 0.2) (layer "F.Cu") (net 3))
 (via (at 164.4015 80.7085) (size 0.6) (drill 0.3) (layers "F.Cu" "B.Cu") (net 3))
 (segment (start 165.1635 80.7085) (end 165.735 81.28) (width 0.2) (layer "B.Cu") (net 3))
 (segment (start 164.4015 80.7085) (end 165.1635 80.7085) (width 0.2) (layer "B.Cu") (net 3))
 (segment (start 167.64 85.68) (end 165.145 83.185) (width 0.2) (layer "B.Cu") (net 27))
 (segment (start 165.145 83.185) (end 160.02 83.185) (width 0.2) (layer "B.Cu") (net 27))
 (segment (start 167.64 86.48) (end 167.64 85.68) (width 0.2) (layer "B.Cu") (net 27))
 (segment (start 160.02 83.185) (end 160.02 81.915) (width 0.2) (layer "B.Cu") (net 27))
 (segment (start 164.91 83.585) (end 158.8725 83.585) (width 0.2) (layer "B.Cu") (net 28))
 (segment (start 167.005 86.48) (end 167.005 85.68) (width 0.2) (layer "B.Cu") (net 28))
 (segment (start 167.005 85.68) (end 164.91 83.585) (width 0.2) (layer "B.Cu") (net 28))
 (segment (start 158.8725 83.585) (end 156.845 81.5575) (width 0.2) (layer "B.Cu") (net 28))
 (segment (start 166.535 82.55) (end 167.005 82.08) (width 0.2) (layer "B.Cu") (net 30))
 (segment (start 167.005 82.08) (end 167.005 81.28) (width 0.2) (layer "B.Cu") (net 30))
 (segment (start 163.175 81.895) (end 163.83 82.55) (width 0.2) (layer "B.Cu") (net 30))
 (segment (start 162.56 81.895) (end 163.175 81.895) (width 0.2) (layer "B.Cu") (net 30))
 (segment (start 163.83 82.55) (end 166.535 82.55) (width 0.2) (layer "B.Cu") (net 30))
 (segment (start 156.718 87.376) (end 156.7 87.358) (width 0.2) (layer "F.Cu") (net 1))
 (segment (start 156.7 87.358) (end 156.7 83.82) (width 0.2) (layer "F.Cu") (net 1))
 (via (at 156.718 87.376) (size 0.6) (drill 0.3) (layers "F.Cu" "B.Cu") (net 1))
 (segment (start 168.275 87.376) (end 168.275 86.48) (width 0.2) (layer "B.Cu") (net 1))
 (segment (start 157.226 87.884) (end 167.767 87.884) (width 0.2) (layer "B.Cu") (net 1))
 (segment (start 156.718 87.376) (end 157.226 87.884) (width 0.2) (layer "B.Cu") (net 1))
 (segment (start 167.767 87.884) (end 168.275 87.376) (width 0.2) (layer "B.Cu") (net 1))
 (segment (start 162.56 79.395) (end 165.285 79.395) (width 0.2) (layer "B.Cu") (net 29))
 (segment (start 165.285 79.395) (end 166.37 80.48) (width 0.2) (layer "B.Cu") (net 29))
 (segment (start 166.37 80.48) (end 166.37 81.28) (width 0.2) (layer "B.Cu") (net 29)))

